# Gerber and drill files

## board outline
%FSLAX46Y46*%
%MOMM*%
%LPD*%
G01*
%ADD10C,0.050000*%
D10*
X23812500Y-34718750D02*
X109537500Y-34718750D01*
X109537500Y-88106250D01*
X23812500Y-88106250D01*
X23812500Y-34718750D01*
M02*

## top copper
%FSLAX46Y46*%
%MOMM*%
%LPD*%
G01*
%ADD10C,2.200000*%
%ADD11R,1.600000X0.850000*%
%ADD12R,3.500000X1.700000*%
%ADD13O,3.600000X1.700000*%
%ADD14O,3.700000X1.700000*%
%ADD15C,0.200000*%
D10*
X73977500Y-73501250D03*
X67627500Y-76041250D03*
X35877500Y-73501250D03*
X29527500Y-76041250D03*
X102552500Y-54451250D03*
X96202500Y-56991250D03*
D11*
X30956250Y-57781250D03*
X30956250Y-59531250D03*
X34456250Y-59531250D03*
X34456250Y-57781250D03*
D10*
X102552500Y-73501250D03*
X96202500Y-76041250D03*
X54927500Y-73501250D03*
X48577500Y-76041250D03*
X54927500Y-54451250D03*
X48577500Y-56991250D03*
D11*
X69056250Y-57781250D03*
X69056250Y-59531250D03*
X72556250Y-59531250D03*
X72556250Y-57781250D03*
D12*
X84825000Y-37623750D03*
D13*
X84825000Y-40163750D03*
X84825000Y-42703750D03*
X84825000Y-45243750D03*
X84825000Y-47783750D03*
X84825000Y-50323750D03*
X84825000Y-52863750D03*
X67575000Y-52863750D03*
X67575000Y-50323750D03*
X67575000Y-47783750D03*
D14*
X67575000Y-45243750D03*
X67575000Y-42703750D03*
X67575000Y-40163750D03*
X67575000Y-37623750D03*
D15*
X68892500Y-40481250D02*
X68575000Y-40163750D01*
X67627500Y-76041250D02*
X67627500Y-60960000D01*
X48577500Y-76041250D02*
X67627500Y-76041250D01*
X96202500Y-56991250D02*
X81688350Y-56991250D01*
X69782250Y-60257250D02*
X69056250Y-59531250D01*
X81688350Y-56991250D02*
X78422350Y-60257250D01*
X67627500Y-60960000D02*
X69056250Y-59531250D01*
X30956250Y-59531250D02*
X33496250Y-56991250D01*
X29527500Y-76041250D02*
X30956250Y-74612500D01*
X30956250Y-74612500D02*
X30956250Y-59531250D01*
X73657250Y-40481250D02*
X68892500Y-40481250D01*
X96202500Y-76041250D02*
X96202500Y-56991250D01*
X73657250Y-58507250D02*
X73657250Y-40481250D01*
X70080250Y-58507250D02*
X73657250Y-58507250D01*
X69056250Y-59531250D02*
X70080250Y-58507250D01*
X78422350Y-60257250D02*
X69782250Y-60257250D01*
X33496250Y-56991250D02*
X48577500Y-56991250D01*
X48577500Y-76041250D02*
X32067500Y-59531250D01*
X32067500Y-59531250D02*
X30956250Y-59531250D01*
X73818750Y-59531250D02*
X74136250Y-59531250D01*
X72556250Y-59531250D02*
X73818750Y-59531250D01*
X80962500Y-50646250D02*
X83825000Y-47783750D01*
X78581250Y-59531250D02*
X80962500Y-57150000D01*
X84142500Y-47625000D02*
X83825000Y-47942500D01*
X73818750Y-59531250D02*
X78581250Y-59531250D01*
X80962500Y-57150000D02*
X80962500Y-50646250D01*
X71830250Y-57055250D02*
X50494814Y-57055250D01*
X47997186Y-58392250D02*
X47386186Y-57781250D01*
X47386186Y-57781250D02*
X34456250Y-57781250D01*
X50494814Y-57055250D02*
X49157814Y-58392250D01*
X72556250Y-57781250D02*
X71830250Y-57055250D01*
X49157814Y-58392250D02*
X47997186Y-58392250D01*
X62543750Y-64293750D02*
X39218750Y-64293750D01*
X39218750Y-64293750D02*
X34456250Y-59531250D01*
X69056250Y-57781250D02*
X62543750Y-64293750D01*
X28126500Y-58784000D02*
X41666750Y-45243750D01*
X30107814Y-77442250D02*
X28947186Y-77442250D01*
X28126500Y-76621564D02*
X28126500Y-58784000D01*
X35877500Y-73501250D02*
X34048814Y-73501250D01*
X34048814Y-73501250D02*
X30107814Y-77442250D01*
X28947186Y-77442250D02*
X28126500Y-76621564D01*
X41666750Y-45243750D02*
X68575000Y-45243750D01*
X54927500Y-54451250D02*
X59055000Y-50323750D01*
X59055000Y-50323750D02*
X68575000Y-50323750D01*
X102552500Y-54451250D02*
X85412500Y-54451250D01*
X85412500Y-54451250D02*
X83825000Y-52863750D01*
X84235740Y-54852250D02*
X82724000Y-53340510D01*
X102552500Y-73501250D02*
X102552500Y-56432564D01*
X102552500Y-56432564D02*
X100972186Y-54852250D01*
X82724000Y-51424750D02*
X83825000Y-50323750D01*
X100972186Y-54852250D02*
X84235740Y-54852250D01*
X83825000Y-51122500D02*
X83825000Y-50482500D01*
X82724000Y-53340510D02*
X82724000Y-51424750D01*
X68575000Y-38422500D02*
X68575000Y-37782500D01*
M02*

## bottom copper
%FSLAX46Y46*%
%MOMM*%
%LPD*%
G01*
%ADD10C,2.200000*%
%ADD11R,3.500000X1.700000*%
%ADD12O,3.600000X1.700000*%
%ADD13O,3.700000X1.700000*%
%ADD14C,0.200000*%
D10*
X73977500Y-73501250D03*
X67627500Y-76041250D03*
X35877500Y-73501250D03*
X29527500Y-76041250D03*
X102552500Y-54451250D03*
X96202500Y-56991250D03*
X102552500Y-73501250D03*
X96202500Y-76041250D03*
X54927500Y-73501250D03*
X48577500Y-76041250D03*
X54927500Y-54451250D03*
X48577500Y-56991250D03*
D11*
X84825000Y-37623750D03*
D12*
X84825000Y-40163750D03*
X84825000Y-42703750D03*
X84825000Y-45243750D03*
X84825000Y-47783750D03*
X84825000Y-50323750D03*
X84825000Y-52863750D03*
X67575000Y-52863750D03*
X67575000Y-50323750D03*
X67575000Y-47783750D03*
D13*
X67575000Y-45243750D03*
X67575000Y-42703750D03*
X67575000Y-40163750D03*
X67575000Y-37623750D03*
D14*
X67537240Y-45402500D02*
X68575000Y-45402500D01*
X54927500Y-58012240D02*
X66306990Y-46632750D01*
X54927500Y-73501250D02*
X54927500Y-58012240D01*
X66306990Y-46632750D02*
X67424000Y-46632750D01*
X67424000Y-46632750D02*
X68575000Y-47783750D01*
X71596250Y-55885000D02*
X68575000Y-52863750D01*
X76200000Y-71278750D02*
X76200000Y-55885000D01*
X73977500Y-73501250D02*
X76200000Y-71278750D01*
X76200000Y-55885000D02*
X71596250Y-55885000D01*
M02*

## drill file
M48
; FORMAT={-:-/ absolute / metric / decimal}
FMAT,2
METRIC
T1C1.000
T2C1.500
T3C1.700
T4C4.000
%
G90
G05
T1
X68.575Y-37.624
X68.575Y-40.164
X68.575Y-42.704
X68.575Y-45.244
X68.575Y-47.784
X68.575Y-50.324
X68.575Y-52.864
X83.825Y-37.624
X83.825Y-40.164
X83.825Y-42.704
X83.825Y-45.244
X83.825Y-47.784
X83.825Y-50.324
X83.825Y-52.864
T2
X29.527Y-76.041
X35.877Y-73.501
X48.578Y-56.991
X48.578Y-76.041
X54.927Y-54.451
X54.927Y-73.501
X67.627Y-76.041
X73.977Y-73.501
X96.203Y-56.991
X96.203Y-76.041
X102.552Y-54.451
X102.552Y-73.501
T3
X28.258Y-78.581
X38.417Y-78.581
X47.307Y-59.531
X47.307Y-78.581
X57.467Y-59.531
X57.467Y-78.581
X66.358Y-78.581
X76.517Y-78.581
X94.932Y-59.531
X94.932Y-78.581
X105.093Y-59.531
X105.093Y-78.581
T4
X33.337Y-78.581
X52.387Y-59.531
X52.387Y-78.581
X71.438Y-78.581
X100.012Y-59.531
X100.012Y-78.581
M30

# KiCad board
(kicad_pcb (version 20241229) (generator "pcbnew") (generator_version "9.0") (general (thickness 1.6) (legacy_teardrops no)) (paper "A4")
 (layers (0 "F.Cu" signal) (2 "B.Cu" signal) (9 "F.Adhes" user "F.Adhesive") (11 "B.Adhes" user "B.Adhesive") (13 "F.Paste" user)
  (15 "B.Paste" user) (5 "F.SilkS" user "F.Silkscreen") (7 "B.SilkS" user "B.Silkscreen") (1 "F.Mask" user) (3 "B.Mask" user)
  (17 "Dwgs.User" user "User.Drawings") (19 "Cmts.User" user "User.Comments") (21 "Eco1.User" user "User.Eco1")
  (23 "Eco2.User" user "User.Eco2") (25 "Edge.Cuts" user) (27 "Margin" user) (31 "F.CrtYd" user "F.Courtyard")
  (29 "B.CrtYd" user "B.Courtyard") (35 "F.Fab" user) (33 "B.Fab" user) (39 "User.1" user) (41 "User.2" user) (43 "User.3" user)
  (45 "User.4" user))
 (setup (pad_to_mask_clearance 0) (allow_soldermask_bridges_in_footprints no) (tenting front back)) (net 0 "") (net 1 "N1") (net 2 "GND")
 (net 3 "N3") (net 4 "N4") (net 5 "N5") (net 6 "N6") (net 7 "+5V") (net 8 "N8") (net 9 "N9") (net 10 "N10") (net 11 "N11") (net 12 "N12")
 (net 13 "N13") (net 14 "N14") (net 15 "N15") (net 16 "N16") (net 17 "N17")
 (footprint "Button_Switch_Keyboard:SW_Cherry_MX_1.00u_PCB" (layer "F.Cu") (at 73.9775 73.50125)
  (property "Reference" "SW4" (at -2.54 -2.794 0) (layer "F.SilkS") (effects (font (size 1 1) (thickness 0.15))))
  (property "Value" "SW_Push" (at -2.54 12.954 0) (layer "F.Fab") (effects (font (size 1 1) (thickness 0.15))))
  (pad "" np_thru_hole circle (at -7.62 5.08) (size 1.7 1.7) (drill 1.7) (layers "*.Cu" "*.Mask"))
  (pad "" np_thru_hole circle (at -2.54 5.08) (size 4 4) (drill 4) (layers "*.Cu" "*.Mask"))
  (pad "" np_thru_hole circle (at 2.54 5.08) (size 1.7 1.7) (drill 1.7) (layers "*.Cu" "*.Mask"))
  (pad "1" thru_hole circle (at 0 0) (size 2.2 2.2) (drill 1.5) (layers "*.Cu" "*.Mask") (remove_unused_layers no) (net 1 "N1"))
  (pad "2" thru_hole circle (at -6.35 2.54) (size 2.2 2.2) (drill 1.5) (layers "*.Cu" "*.Mask") (remove_unused_layers no) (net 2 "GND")))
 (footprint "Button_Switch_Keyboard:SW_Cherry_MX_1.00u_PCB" (layer "F.Cu") (at 35.8775 73.50125)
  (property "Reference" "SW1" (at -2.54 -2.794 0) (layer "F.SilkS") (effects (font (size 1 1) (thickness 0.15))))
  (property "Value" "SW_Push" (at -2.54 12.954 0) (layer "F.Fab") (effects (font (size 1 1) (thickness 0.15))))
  (pad "" np_thru_hole circle (at -7.62 5.08) (size 1.7 1.7) (drill 1.7) (layers "*.Cu" "*.Mask"))
  (pad "" np_thru_hole circle (at -2.54 5.08) (size 4 4) (drill 4) (layers "*.Cu" "*.Mask"))
  (pad "" np_thru_hole circle (at 2.54 5.08) (size 1.7 1.7) (drill 1.7) (layers "*.Cu" "*.Mask"))
  (pad "1" thru_hole circle (at 0 0) (size 2.2 2.2) (drill 1.5) (layers "*.Cu" "*.Mask") (remove_unused_layers no) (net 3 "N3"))
  (pad "2" thru_hole circle (at -6.35 2.54) (size 2.2 2.2) (drill 1.5) (layers "*.Cu" "*.Mask") (remove_unused_layers no) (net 2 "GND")))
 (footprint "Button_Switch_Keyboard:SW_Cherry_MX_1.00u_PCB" (layer "F.Cu") (at 102.5525 54.45125)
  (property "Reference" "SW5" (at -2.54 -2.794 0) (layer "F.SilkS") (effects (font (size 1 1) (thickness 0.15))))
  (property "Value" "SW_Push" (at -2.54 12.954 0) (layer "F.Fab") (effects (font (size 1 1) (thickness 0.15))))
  (pad "" np_thru_hole circle (at -7.62 5.08) (size 1.7 1.7) (drill 1.7) (layers "*.Cu" "*.Mask"))
  (pad "" np_thru_hole circle (at -2.54 5.08) (size 4 4) (drill 4) (layers "*.Cu" "*.Mask"))
  (pad "" np_thru_hole circle (at 2.54 5.08) (size 1.7 1.7) (drill 1.7) (layers "*.Cu" "*.Mask"))
  (pad "1" thru_hole circle (at 0 0) (size 2.2 2.2) (drill 1.5) (layers "*.Cu" "*.Mask") (remove_unused_layers no) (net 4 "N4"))
  (pad "2" thru_hole circle (at -6.35 2.54) (size 2.2 2.2) (drill 1.5) (layers "*.Cu" "*.Mask") (remove_unused_layers no) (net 2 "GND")))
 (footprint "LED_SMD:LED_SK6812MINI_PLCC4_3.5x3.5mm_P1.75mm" (layer "F.Cu") (at 32.70625 58.65625)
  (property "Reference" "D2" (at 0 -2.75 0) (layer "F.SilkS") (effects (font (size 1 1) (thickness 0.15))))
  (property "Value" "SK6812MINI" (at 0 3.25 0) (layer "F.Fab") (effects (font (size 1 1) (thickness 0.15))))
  (pad "1" smd rect (at -1.75 -0.875) (size 1.6 0.85) (layers "F.Cu" "F.Mask" "F.Paste") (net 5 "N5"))
  (pad "2" smd rect (at -1.75 0.875) (size 1.6 0.85) (layers "F.Cu" "F.Mask" "F.Paste") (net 2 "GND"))
  (pad "3" smd rect (at 1.75 0.875) (size 1.6 0.85) (layers "F.Cu" "F.Mask" "F.Paste") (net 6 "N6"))
  (pad "4" smd rect (at 1.75 -0.875) (size 1.6 0.85) (layers "F.Cu" "F.Mask" "F.Paste") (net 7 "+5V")))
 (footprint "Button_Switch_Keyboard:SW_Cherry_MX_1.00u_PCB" (layer "F.Cu") (at 102.5525 73.50125)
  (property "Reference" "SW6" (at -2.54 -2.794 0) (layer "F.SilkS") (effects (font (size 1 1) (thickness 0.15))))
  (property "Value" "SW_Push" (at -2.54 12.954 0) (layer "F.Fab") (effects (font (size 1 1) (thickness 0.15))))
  (pad "" np_thru_hole circle (at -7.62 5.08) (size 1.7 1.7) (drill 1.7) (layers "*.Cu" "*.Mask"))
  (pad "" np_thru_hole circle (at -2.54 5.08) (size 4 4) (drill 4) (layers "*.Cu" "*.Mask"))
  (pad "" np_thru_hole circle (at 2.54 5.08) (size 1.7 1.7) (drill 1.7) (layers "*.Cu" "*.Mask"))
  (pad "1" thru_hole circle (at 0 0) (size 2.2 2.2) (drill 1.5) (layers "*.Cu" "*.Mask") (remove_unused_layers no) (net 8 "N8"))
  (pad "2" thru_hole circle (at -6.35 2.54) (size 2.2 2.2) (drill 1.5) (layers "*.Cu" "*.Mask") (remove_unused_layers no) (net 2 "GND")))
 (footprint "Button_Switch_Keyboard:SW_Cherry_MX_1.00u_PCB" (layer "F.Cu") (at 54.9275 73.50125)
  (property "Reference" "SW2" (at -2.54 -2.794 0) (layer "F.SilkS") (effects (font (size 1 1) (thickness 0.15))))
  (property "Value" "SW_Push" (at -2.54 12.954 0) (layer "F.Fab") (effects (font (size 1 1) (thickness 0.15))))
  (pad "" np_thru_hole circle (at -7.62 5.08) (size 1.7 1.7) (drill 1.7) (layers "*.Cu" "*.Mask"))
  (pad "" np_thru_hole circle (at -2.54 5.08) (size 4 4) (drill 4) (layers "*.Cu" "*.Mask"))
  (pad "" np_thru_hole circle (at 2.54 5.08) (size 1.7 1.7) (drill 1.7) (layers "*.Cu" "*.Mask"))
  (pad "1" thru_hole circle (at 0 0) (size 2.2 2.2) (drill 1.5) (layers "*.Cu" "*.Mask") (remove_unused_layers no) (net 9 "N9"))
  (pad "2" thru_hole circle (at -6.35 2.54) (size 2.2 2.2) (drill 1.5) (layers "*.Cu" "*.Mask") (remove_unused_layers no) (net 2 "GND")))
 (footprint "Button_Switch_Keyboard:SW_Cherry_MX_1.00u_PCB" (layer "F.Cu") (at 54.9275 54.45125)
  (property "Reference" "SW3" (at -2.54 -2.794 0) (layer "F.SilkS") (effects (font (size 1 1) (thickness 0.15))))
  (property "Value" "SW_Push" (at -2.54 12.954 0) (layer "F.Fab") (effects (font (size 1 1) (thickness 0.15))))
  (pad "" np_thru_hole circle (at -7.62 5.08) (size 1.7 1.7) (drill 1.7) (layers "*.Cu" "*.Mask"))
  (pad "" np_thru_hole circle (at -2.54 5.08) (size 4 4) (drill 4) (layers "*.Cu" "*.Mask"))
  (pad "" np_thru_hole circle (at 2.54 5.08) (size 1.7 1.7) (drill 1.7) (layers "*.Cu" "*.Mask"))
  (pad "1" thru_hole circle (at 0 0) (size 2.2 2.2) (drill 1.5) (layers "*.Cu" "*.Mask") (remove_unused_layers no) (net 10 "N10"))
  (pad "2" thru_hole circle (at -6.35 2.54) (size 2.2 2.2) (drill 1.5) (layers "*.Cu" "*.Mask") (remove_unused_layers no) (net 2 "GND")))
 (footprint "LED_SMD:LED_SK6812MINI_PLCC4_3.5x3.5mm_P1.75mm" (layer "F.Cu") (at 70.80625 58.65625)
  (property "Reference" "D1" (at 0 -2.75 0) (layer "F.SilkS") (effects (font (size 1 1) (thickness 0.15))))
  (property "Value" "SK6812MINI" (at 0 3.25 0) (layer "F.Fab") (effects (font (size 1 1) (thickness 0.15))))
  (pad "1" smd rect (at -1.75 -0.875) (size 1.6 0.85) (layers "F.Cu" "F.Mask" "F.Paste") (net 6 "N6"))
  (pad "2" smd rect (at -1.75 0.875) (size 1.6 0.85) (layers "F.Cu" "F.Mask" "F.Paste") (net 2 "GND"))
  (pad "3" smd rect (at 1.75 0.875) (size 1.6 0.85) (layers "F.Cu" "F.Mask" "F.Paste") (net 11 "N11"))
  (pad "4" smd rect (at 1.75 -0.875) (size 1.6 0.85) (layers "F.Cu" "F.Mask" "F.Paste") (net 7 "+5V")))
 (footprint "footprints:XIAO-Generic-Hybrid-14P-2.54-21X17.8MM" (layer "B.Cu") (at 76.2 45.24375 180)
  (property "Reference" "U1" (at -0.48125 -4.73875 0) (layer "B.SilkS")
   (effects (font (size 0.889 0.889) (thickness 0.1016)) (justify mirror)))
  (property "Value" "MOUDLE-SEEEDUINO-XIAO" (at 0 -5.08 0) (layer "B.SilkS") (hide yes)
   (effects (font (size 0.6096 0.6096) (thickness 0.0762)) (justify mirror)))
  (pad "1" thru_hole rect (at -7.625 7.62 180) (size 3.5 1.7) (drill 1 (offset -1 0)) (layers "*.Cu" "*.Mask") (remove_unused_layers no)
   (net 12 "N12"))
  (pad "2" thru_hole oval (at -7.625 5.08 180) (size 3.6 1.7) (drill 1 (offset -1 0)) (layers "*.Cu" "*.Mask") (remove_unused_layers no)
   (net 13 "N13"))
  (pad "3" thru_hole oval (at -7.625 2.54 180) (size 3.6 1.7) (drill 1 (offset -1 0)) (layers "*.Cu" "*.Mask") (remove_unused_layers no)
   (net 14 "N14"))
  (pad "4" thru_hole oval (at -7.625 0 180) (size 3.6 1.7) (drill 1 (offset -1 0)) (layers "*.Cu" "*.Mask") (remove_unused_layers no)
   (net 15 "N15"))
  (pad "5" thru_hole oval (at -7.625 -2.54 180) (size 3.6 1.7) (drill 1 (offset -1 0)) (layers "*.Cu" "*.Mask") (remove_unused_layers no)
   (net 11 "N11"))
  (pad "6" thru_hole oval (at -7.625 -5.08) (size 3.6 1.7) (drill 1 (offset 1 0)) (layers "*.Cu" "*.Mask") (remove_unused_layers no)
   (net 8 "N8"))
  (pad "7" thru_hole oval (at -7.625 -7.62 180) (size 3.6 1.7) (drill 1 (offset -1 0)) (layers "*.Cu" "*.Mask") (remove_unused_layers no)
   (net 4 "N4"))
  (pad "8" thru_hole oval (at 7.625 -7.62 180) (size 3.6 1.7) (drill 1 (offset 1 0)) (layers "*.Cu" "*.Mask") (remove_unused_layers no)
   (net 1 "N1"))
  (pad "9" thru_hole oval (at 7.625 -5.08 180) (size 3.6 1.7) (drill 1 (offset 1 0)) (layers "*.Cu" "*.Mask") (remove_unused_layers no)
   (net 10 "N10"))
  (pad "10" thru_hole oval (at 7.625 -2.54 180) (size 3.6 1.7) (drill 1 (offset 1 0)) (layers "*.Cu" "*.Mask") (remove_unused_layers no)
   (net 9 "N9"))
  (pad "11" thru_hole oval (at 7.625 0 180) (size 3.7 1.7) (drill 1 (offset 1 0)) (layers "*.Cu" "*.Mask") (remove_unused_layers no)
   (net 3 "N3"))
  (pad "12" thru_hole oval (at 7.625 2.54 180) (size 3.7 1.7) (drill 1 (offset 1 0)) (layers "*.Cu" "*.Mask") (remove_unused_layers no)
   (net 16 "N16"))
  (pad "13" thru_hole oval (at 7.625 5.08 180) (size 3.7 1.7) (drill 1 (offset 1 0)) (layers "*.Cu" "*.Mask") (remove_unused_layers no)
   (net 2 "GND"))
  (pad "14" thru_hole oval (at 7.625 7.62 180) (size 3.7 1.7) (drill 1 (offset 1 0)) (layers "*.Cu" "*.Mask") (remove_unused_layers no)
   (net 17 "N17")))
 (gr_rect (start 23.8125 34.71875) (end 109.5375 88.10625) (stroke (width 0.05) (type default)) (fill no) (layer "Edge.Cuts"))
 (segment (start 68.8925 40.48125) (end 68.575 40.16375) (width 0.2) (layer "F.Cu") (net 2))
 (segment (start 67.6275 76.04125) (end 67.6275 60.96) (width 0.2) (layer "F.Cu") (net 2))
 (segment (start 48.5775 76.04125) (end 67.6275 76.04125) (width 0.2) (layer "F.Cu") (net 2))
 (segment (start 96.2025 56.99125) (end 81.68835 56.99125) (width 0.2) (layer "F.Cu") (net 2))
 (segment (start 69.78225 60.25725) (end 69.05625 59.53125) (width 0.2) (layer "F.Cu") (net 2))
 (segment (start 81.68835 56.99125) (end 78.42235 60.25725) (width 0.2) (layer "F.Cu") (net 2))
 (segment (start 67.6275 60.96) (end 69.05625 59.53125) (width 0.2) (layer "F.Cu") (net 2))
 (segment (start 30.95625 59.53125) (end 33.49625 56.99125) (width 0.2) (layer "F.Cu") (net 2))
 (segment (start 29.5275 76.04125) (end 30.95625 74.6125) (width 0.2) (layer "F.Cu") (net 2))
 (segment (start 30.95625 74.6125) (end 30.95625 59.53125) (width 0.2) (layer "F.Cu") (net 2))
 (segment (start 73.65725 40.48125) (end 68.8925 40.48125) (width 0.2) (layer "F.Cu") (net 2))
 (segment (start 96.2025 76.04125) (end 96.2025 56.99125) (width 0.2) (layer "F.Cu") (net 2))
 (segment (start 73.65725 58.50725) (end 73.65725 40.48125) (width 0.2) (layer "F.Cu") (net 2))
 (segment (start 70.08025 58.50725) (end 73.65725 58.50725) (width 0.2) (layer "F.Cu") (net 2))
 (segment (start 69.05625 59.53125) (end 70.08025 58.50725) (width 0.2) (layer "F.Cu") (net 2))
 (segment (start 78.42235 60.25725) (end 69.78225 60.25725) (width 0.2) (layer "F.Cu") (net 2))
 (segment (start 33.49625 56.99125) (end 48.5775 56.99125) (width 0.2) (layer "F.Cu") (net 2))
 (segment (start 48.5775 76.04125) (end 32.0675 59.53125) (width 0.2) (layer "F.Cu") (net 2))
 (segment (start 32.0675 59.53125) (end 30.95625 59.53125) (width 0.2) (layer "F.Cu") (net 2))
 (segment (start 73.81875 59.53125) (end 74.13625 59.53125) (width 0.2) (layer "F.Cu") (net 11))
 (segment (start 72.55625 59.53125) (end 73.81875 59.53125) (width 0.2) (layer "F.Cu") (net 11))
 (segment (start 80.9625 50.64625) (end 83.825 47.78375) (width 0.2) (layer "F.Cu") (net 11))
 (segment (start 78.58125 59.53125) (end 80.9625 57.15) (width 0.2) (layer "F.Cu") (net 11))
 (segment (start 84.1425 47.625) (end 83.825 47.9425) (width 0.2) (layer "F.Cu") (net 11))
 (segment (start 73.81875 59.53125) (end 78.58125 59.53125) (width 0.2) (layer "F.Cu") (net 11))
 (segment (start 80.9625 57.15) (end 80.9625 50.64625) (width 0.2) (layer "F.Cu") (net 11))
 (segment (start 71.83025 57.05525) (end 50.494814 57.05525) (width 0.2) (layer "F.Cu") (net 7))
 (segment (start 47.997186 58.39225) (end 47.386186 57.78125) (width 0.2) (layer "F.Cu") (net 7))
 (segment (start 47.386186 57.78125) (end 34.45625 57.78125) (width 0.2) (layer "F.Cu") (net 7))
 (segment (start 50.494814 57.05525) (end 49.157814 58.39225) (width 0.2) (layer "F.Cu") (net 7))
 (segment (start 72.55625 57.78125) (end 71.83025 57.05525) (width 0.2) (layer "F.Cu") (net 7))
 (segment (start 49.157814 58.39225) (end 47.997186 58.39225) (width 0.2) (layer "F.Cu") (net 7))
 (segment (start 62.54375 64.29375) (end 39.21875 64.29375) (width 0.2) (layer "F.Cu") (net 6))
 (segment (start 39.21875 64.29375) (end 34.45625 59.53125) (width 0.2) (layer "F.Cu") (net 6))
 (segment (start 69.05625 57.78125) (end 62.54375 64.29375) (width 0.2) (layer "F.Cu") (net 6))
 (segment (start 28.1265 58.784) (end 41.66675 45.24375) (width 0.2) (layer "F.Cu") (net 3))
 (segment (start 30.107814 77.44225) (end 28.947186 77.44225) (width 0.2) (layer "F.Cu") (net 3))
 (segment (start 28.1265 76.621564) (end 28.1265 58.784) (width 0.2) (layer "F.Cu") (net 3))
 (segment (start 35.8775 73.50125) (end 34.048814 73.50125) (width 0.2) (layer "F.Cu") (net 3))
 (segment (start 34.048814 73.50125) (end 30.107814 77.44225) (width 0.2) (layer "F.Cu") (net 3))
 (segment (start 28.947186 77.44225) (end 28.1265 76.621564) (width 0.2) (layer "F.Cu") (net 3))
 (segment (start 41.66675 45.24375) (end 68.575 45.24375) (width 0.2) (layer "F.Cu") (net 3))
 (segment (start 67.53724 45.4025) (end 68.575 45.4025) (width 0.2) (layer "B.Cu") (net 3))
 (segment (start 54.9275 58.01224) (end 66.30699 46.63275) (width 0.2) (layer "B.Cu") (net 9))
 (segment (start 54.9275 73.50125) (end 54.9275 58.01224) (width 0.2) (layer "B.Cu") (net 9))
 (segment (start 66.30699 46.63275) (end 67.424 46.63275) (width 0.2) (layer "B.Cu") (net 9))
 (segment (start 67.424 46.63275) (end 68.575 47.78375) (width 0.2) (layer "B.Cu") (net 9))
 (segment (start 54.9275 54.45125) (end 59.055 50.32375) (width 0.2) (layer "F.Cu") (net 10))
 (segment (start 59.055 50.32375) (end 68.575 50.32375) (width 0.2) (layer "F.Cu") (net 10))
 (segment (start 71.59625 55.885) (end 68.575 52.86375) (width 0.2) (layer "B.Cu") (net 1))
 (segment (start 76.2 71.27875) (end 76.2 55.885) (width 0.2) (layer "B.Cu") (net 1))
 (segment (start 73.9775 73.50125) (end 76.2 71.27875) (width 0.2) (layer "B.Cu") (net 1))
 (segment (start 76.2 55.885) (end 71.59625 55.885) (width 0.2) (layer "B.Cu") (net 1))
 (segment (start 102.5525 54.45125) (end 85.4125 54.45125) (width 0.2) (layer "F.Cu") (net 4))
 (segment (start 85.4125 54.45125) (end 83.825 52.86375) (width 0.2) (layer "F.Cu") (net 4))
 (segment (start 84.23574 54.85225) (end 82.724 53.34051) (width 0.2) (layer "F.Cu") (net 8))
 (segment (start 102.5525 73.50125) (end 102.5525 56.432564) (width 0.2) (layer "F.Cu") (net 8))
 (segment (start 102.5525 56.432564) (end 100.972186 54.85225) (width 0.2) (layer "F.Cu") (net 8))
 (segment (start 82.724 51.42475) (end 83.825 50.32375) (width 0.2) (layer "F.Cu") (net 8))
 (segment (start 100.972186 54.85225) (end 84.23574 54.85225) (width 0.2) (layer "F.Cu") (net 8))
 (segment (start 83.825 51.1225) (end 83.825 50.4825) (width 0.2) (layer "F.Cu") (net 8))
 (segment (start 82.724 53.34051) (end 82.724 51.42475) (width 0.2) (layer "F.Cu") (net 8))
 (segment (start 68.575 38.4225) (end 68.575 37.7825) (width 0.2) (layer "F.Cu") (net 17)))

